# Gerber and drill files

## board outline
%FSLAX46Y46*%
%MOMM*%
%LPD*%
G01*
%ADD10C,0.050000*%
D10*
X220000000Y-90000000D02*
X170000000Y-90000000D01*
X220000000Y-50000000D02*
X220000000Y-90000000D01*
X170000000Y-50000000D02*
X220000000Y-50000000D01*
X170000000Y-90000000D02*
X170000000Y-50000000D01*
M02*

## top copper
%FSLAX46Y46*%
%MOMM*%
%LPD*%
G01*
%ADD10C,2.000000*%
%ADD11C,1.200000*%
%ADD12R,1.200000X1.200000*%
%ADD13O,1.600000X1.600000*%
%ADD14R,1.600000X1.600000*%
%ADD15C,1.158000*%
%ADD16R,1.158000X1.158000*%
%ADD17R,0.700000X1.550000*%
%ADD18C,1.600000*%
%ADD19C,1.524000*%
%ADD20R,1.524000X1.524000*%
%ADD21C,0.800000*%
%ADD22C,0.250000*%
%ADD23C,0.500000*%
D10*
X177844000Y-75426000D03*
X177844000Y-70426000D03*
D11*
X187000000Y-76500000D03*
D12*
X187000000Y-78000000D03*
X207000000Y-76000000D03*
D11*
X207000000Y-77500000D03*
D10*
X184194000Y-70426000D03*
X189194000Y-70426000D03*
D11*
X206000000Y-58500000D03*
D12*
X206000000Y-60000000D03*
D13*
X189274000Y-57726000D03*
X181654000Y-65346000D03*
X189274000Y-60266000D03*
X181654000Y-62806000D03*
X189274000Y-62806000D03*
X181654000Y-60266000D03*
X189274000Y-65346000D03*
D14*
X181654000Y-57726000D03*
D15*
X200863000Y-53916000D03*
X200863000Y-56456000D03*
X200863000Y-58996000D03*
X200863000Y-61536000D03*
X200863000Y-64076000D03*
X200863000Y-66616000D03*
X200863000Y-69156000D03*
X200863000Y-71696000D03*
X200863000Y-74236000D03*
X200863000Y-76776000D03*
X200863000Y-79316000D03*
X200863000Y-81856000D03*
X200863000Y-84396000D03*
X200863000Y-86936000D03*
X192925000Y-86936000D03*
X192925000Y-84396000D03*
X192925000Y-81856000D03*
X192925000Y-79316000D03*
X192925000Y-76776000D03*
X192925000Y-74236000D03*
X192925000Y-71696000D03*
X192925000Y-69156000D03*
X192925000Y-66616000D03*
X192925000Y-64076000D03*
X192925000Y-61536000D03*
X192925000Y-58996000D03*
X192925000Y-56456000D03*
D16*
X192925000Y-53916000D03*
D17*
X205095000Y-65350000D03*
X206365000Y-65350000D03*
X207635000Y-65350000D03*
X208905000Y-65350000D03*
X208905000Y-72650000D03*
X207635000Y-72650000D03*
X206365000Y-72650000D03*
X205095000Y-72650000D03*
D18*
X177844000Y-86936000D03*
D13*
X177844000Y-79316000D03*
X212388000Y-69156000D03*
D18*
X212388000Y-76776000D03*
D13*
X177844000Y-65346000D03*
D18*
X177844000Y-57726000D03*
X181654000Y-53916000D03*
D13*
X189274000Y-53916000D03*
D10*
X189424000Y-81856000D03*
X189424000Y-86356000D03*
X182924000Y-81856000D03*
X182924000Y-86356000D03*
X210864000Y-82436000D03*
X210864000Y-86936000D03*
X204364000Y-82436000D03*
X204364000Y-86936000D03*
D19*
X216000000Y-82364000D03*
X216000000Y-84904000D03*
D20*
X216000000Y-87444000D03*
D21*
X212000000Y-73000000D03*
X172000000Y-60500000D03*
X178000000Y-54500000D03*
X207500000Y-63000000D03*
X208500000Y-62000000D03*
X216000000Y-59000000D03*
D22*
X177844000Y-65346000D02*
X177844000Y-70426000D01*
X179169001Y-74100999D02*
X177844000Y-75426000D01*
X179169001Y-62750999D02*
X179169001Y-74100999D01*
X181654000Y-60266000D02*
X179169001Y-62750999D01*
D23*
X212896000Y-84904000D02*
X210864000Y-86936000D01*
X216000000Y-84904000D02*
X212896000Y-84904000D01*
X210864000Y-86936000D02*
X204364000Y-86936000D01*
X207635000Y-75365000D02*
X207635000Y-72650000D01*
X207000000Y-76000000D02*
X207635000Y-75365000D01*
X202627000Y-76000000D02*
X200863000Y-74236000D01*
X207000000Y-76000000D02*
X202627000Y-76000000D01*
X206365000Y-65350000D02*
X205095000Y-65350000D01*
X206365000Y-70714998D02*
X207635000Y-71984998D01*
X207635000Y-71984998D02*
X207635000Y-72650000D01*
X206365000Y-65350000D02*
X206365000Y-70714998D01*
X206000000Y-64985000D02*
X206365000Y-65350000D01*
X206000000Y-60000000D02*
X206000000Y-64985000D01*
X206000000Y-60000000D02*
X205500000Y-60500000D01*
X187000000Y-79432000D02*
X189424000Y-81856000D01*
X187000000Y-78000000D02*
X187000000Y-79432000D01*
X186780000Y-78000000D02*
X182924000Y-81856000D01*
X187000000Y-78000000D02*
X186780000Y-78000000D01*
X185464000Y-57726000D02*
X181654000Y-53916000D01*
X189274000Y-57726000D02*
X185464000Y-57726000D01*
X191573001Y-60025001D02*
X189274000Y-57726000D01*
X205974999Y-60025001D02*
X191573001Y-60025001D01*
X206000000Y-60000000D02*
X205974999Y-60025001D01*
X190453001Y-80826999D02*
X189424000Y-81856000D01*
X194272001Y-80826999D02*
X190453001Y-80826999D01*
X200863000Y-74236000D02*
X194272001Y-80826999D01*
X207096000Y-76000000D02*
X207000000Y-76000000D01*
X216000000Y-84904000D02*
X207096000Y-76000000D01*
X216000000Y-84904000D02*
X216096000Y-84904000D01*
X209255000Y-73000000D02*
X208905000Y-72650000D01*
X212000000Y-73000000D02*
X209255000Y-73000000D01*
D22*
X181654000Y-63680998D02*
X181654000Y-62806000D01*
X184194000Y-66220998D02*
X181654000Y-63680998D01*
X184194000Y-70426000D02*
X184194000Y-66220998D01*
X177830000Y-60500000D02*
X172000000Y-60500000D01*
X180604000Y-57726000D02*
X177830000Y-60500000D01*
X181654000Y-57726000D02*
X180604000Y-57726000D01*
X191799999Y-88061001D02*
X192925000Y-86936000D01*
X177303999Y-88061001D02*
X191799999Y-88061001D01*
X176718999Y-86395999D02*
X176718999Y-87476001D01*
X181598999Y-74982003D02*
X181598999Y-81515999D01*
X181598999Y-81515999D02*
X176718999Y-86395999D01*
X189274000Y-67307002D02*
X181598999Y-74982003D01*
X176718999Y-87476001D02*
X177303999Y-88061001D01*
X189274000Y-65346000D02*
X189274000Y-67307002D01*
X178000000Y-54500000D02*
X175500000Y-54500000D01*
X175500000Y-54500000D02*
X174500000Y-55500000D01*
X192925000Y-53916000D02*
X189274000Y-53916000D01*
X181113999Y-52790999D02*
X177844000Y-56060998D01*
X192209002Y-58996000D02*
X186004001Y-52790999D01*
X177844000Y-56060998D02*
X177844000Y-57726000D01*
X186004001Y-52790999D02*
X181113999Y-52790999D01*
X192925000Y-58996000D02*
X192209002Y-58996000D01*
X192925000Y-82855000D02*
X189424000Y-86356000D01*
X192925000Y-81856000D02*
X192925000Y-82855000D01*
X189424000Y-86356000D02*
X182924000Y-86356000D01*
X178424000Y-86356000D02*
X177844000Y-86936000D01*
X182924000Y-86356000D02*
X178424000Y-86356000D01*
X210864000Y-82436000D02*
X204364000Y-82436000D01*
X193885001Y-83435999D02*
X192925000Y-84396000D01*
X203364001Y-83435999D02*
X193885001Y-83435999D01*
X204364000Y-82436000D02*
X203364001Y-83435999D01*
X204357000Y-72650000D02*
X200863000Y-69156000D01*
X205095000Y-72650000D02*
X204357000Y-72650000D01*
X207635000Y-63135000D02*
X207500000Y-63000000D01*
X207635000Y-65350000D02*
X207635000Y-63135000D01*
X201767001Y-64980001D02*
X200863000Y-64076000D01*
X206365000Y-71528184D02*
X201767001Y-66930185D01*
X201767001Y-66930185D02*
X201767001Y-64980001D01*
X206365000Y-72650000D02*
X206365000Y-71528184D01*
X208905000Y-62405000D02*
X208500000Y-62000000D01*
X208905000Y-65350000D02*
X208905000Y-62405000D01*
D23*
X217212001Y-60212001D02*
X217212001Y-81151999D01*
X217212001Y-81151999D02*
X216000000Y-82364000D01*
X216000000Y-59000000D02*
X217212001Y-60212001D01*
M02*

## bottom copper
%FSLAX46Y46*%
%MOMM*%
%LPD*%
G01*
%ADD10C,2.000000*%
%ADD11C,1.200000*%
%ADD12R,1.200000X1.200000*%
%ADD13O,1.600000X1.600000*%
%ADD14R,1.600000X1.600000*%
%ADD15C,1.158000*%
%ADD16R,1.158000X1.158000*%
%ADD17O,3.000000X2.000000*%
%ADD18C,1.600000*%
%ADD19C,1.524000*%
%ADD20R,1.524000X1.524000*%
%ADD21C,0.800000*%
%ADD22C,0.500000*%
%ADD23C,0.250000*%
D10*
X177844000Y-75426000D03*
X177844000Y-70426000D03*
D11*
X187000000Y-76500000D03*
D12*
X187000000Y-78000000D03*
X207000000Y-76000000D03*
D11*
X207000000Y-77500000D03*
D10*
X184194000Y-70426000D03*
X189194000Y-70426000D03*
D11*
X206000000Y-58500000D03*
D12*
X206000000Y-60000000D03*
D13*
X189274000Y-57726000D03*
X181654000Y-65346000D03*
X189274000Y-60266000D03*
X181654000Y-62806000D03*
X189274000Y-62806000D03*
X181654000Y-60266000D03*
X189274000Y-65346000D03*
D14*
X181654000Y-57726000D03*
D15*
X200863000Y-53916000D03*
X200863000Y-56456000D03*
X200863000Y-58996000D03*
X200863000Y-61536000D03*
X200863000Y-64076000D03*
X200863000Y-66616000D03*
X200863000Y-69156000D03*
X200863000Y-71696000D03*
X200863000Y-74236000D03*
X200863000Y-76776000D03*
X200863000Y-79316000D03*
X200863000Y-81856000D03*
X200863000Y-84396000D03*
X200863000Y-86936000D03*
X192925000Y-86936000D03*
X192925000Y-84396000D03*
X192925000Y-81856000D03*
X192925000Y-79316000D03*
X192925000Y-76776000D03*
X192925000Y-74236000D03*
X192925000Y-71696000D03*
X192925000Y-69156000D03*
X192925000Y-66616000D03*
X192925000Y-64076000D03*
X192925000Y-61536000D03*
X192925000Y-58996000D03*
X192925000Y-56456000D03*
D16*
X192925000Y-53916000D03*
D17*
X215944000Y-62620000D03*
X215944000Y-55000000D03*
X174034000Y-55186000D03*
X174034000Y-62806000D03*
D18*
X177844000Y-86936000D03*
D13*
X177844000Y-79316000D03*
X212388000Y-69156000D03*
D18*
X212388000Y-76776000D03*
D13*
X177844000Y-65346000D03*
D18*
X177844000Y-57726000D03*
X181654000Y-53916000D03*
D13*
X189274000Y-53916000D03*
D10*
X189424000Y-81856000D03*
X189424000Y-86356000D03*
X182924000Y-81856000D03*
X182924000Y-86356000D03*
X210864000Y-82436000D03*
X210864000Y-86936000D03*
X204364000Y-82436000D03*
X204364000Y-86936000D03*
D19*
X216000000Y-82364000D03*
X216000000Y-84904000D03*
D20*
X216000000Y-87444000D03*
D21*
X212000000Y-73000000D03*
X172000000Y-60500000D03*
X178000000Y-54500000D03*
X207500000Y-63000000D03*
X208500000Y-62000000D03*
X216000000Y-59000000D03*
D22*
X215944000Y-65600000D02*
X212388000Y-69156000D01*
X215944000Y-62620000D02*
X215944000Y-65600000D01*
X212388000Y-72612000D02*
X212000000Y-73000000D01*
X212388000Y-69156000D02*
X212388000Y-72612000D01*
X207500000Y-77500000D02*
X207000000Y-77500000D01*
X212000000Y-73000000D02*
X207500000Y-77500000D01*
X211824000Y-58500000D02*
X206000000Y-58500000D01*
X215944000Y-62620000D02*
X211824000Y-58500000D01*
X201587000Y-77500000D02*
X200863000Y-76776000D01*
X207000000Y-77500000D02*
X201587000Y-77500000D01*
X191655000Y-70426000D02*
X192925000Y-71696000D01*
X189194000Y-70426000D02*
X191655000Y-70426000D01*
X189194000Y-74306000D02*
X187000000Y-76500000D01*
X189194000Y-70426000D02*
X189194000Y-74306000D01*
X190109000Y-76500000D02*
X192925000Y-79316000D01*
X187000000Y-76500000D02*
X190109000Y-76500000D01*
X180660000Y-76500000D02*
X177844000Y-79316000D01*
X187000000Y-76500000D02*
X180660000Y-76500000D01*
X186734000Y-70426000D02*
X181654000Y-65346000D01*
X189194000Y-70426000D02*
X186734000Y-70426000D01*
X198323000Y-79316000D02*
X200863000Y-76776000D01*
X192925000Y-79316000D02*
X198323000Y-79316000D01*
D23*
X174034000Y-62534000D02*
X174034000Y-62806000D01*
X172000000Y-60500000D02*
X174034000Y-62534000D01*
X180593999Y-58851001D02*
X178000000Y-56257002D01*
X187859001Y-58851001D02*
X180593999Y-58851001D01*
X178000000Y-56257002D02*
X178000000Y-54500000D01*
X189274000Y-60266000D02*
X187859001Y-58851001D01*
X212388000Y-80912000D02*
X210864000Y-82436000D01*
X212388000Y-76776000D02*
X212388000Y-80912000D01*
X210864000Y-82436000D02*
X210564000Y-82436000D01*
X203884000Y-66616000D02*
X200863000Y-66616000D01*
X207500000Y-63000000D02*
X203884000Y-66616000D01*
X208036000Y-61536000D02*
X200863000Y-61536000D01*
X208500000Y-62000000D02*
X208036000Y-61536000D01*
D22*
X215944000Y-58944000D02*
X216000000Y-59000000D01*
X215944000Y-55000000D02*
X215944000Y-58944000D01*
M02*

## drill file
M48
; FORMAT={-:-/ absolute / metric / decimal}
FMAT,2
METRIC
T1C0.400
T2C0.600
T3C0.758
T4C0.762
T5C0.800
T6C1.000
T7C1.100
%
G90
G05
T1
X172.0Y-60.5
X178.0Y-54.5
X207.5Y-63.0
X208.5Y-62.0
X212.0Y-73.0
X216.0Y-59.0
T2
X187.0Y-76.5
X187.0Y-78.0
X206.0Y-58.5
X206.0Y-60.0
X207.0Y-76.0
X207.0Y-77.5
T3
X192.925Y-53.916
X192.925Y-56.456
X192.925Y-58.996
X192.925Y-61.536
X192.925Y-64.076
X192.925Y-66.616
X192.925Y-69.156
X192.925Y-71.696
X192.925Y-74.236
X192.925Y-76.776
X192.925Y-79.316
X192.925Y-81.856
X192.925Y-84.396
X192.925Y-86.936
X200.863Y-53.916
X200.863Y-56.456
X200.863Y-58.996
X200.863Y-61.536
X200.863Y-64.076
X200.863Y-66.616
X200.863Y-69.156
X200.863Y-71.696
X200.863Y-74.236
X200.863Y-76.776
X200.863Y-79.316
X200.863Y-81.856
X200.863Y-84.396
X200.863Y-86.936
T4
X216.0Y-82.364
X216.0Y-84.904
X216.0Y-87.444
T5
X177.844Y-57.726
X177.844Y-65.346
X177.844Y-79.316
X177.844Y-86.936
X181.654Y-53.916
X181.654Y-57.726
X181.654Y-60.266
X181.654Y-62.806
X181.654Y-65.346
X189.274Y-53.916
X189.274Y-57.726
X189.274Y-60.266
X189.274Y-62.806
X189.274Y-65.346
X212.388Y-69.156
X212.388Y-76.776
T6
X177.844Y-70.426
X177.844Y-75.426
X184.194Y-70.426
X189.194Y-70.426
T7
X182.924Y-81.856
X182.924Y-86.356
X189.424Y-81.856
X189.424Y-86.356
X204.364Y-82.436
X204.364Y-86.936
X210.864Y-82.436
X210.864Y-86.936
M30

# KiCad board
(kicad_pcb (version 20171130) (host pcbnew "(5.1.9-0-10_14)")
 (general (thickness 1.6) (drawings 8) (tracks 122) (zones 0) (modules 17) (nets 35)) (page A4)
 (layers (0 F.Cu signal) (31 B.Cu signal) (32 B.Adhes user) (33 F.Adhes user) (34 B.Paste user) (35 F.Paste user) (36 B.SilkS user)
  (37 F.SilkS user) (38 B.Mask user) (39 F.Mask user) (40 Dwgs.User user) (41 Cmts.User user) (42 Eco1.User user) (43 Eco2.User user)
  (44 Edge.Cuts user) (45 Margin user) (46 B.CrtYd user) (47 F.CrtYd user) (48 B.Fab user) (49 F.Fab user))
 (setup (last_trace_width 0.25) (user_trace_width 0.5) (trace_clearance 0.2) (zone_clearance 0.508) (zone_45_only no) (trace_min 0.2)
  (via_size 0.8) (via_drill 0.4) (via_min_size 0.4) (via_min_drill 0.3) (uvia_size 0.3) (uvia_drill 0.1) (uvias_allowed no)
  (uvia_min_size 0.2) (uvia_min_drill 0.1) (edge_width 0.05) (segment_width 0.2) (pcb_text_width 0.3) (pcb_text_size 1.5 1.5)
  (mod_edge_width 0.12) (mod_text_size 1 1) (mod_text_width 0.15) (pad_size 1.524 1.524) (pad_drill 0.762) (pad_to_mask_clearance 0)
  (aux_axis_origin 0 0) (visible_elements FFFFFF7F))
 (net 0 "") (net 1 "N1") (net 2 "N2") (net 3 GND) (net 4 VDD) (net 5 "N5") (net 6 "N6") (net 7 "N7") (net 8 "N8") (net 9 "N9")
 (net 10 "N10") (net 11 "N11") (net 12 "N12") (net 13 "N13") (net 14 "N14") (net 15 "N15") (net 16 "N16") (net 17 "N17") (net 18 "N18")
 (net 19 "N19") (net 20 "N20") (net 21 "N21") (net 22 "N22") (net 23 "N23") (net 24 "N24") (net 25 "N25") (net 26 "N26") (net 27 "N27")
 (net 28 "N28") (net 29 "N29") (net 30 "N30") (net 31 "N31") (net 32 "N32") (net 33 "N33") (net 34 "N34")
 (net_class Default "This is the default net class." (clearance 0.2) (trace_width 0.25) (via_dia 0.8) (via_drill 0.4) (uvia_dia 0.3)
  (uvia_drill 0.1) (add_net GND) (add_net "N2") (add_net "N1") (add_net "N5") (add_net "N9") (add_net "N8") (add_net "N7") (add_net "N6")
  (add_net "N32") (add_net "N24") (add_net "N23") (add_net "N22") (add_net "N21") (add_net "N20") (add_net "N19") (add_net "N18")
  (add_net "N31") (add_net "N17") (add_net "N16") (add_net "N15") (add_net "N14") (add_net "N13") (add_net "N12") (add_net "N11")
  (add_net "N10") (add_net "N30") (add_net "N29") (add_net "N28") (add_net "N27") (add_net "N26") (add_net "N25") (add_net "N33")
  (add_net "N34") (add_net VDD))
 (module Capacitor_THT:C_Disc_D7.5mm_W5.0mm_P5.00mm (layer F.Cu) (at 177.844 70.426 270)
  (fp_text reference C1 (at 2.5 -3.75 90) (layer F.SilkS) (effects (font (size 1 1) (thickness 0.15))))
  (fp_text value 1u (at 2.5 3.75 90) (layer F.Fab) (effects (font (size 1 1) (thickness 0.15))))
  (pad 2 thru_hole circle (at 5 0 270) (size 2 2) (drill 1) (layers *.Cu *.Mask) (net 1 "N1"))
  (pad 1 thru_hole circle (at 0 0 270) (size 2 2) (drill 1) (layers *.Cu *.Mask) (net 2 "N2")))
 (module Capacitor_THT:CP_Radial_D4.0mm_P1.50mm (layer F.Cu) (at 187 78 90)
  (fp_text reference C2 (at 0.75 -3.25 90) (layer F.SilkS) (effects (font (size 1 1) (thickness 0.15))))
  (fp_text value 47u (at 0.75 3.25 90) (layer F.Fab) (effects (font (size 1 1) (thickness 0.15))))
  (pad 2 thru_hole circle (at 1.5 0 90) (size 1.2 1.2) (drill 0.6) (layers *.Cu *.Mask) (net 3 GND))
  (pad 1 thru_hole rect (at 0 0 90) (size 1.2 1.2) (drill 0.6) (layers *.Cu *.Mask) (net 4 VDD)))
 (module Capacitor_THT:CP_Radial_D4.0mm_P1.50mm (layer F.Cu) (at 207 76 270)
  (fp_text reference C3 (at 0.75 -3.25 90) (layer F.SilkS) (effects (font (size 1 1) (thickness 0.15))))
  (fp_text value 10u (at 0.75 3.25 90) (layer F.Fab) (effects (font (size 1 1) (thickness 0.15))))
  (pad 1 thru_hole rect (at 0 0 270) (size 1.2 1.2) (drill 0.6) (layers *.Cu *.Mask) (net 4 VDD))
  (pad 2 thru_hole circle (at 1.5 0 270) (size 1.2 1.2) (drill 0.6) (layers *.Cu *.Mask) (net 3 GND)))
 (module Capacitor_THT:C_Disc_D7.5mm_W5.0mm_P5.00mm (layer F.Cu) (at 184.194 70.426)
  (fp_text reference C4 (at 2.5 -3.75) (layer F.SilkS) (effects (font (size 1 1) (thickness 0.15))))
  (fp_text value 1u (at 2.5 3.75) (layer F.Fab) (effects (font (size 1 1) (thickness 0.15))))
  (pad 1 thru_hole circle (at 0 0) (size 2 2) (drill 1) (layers *.Cu *.Mask) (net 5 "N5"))
  (pad 2 thru_hole circle (at 5 0) (size 2 2) (drill 1) (layers *.Cu *.Mask) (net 3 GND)))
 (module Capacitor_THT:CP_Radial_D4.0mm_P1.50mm (layer F.Cu) (at 206 60 90)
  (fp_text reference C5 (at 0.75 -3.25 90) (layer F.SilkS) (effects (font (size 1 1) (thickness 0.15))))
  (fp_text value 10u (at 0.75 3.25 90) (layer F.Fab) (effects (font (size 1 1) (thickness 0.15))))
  (pad 2 thru_hole circle (at 1.5 0 90) (size 1.2 1.2) (drill 0.6) (layers *.Cu *.Mask) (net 3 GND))
  (pad 1 thru_hole rect (at 0 0 90) (size 1.2 1.2) (drill 0.6) (layers *.Cu *.Mask) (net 4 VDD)))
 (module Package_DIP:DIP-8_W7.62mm (layer F.Cu) (at 181.654 57.726)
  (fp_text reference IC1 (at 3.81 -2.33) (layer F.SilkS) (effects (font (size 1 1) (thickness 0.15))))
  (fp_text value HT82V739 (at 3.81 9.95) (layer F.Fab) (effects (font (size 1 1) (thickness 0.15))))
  (pad 8 thru_hole oval (at 7.62 0) (size 1.6 1.6) (drill 0.8) (layers *.Cu *.Mask) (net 4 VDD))
  (pad 4 thru_hole oval (at 0 7.62) (size 1.6 1.6) (drill 0.8) (layers *.Cu *.Mask) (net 3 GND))
  (pad 7 thru_hole oval (at 7.62 2.54) (size 1.6 1.6) (drill 0.8) (layers *.Cu *.Mask) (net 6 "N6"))
  (pad 3 thru_hole oval (at 0 5.08) (size 1.6 1.6) (drill 0.8) (layers *.Cu *.Mask) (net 5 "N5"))
  (pad 6 thru_hole oval (at 7.62 5.08) (size 1.6 1.6) (drill 0.8) (layers *.Cu *.Mask) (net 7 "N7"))
  (pad 2 thru_hole oval (at 0 2.54) (size 1.6 1.6) (drill 0.8) (layers *.Cu *.Mask) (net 1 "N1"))
  (pad 5 thru_hole oval (at 7.62 7.62) (size 1.6 1.6) (drill 0.8) (layers *.Cu *.Mask) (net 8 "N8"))
  (pad 1 thru_hole rect (at 0 0) (size 1.6 1.6) (drill 0.8) (layers *.Cu *.Mask) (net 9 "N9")))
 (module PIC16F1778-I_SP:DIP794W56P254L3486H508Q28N (layer F.Cu) (at 196.894 70.426)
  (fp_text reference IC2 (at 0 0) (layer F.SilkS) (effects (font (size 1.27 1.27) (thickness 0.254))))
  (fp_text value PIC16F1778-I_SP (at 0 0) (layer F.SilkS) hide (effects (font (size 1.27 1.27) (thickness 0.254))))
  (pad 28 thru_hole circle (at 3.969 -16.51 90) (size 1.158 1.158) (drill 0.758) (layers *.Cu *.Mask F.SilkS) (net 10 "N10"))
  (pad 27 thru_hole circle (at 3.969 -13.97 90) (size 1.158 1.158) (drill 0.758) (layers *.Cu *.Mask F.SilkS) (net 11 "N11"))
  (pad 26 thru_hole circle (at 3.969 -11.43 90) (size 1.158 1.158) (drill 0.758) (layers *.Cu *.Mask F.SilkS) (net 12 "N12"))
  (pad 25 thru_hole circle (at 3.969 -8.89 90) (size 1.158 1.158) (drill 0.758) (layers *.Cu *.Mask F.SilkS) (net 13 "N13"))
  (pad 24 thru_hole circle (at 3.969 -6.35 90) (size 1.158 1.158) (drill 0.758) (layers *.Cu *.Mask F.SilkS) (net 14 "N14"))
  (pad 23 thru_hole circle (at 3.969 -3.81 90) (size 1.158 1.158) (drill 0.758) (layers *.Cu *.Mask F.SilkS) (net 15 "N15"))
  (pad 22 thru_hole circle (at 3.969 -1.27 90) (size 1.158 1.158) (drill 0.758) (layers *.Cu *.Mask F.SilkS) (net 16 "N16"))
  (pad 21 thru_hole circle (at 3.969 1.27 90) (size 1.158 1.158) (drill 0.758) (layers *.Cu *.Mask F.SilkS) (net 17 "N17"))
  (pad 20 thru_hole circle (at 3.969 3.81 90) (size 1.158 1.158) (drill 0.758) (layers *.Cu *.Mask F.SilkS) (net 4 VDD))
  (pad 19 thru_hole circle (at 3.969 6.35 90) (size 1.158 1.158) (drill 0.758) (layers *.Cu *.Mask F.SilkS) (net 3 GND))
  (pad 18 thru_hole circle (at 3.969 8.89 90) (size 1.158 1.158) (drill 0.758) (layers *.Cu *.Mask F.SilkS) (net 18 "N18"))
  (pad 17 thru_hole circle (at 3.969 11.43 90) (size 1.158 1.158) (drill 0.758) (layers *.Cu *.Mask F.SilkS) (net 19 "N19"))
  (pad 16 thru_hole circle (at 3.969 13.97 90) (size 1.158 1.158) (drill 0.758) (layers *.Cu *.Mask F.SilkS) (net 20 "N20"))
  (pad 15 thru_hole circle (at 3.969 16.51 90) (size 1.158 1.158) (drill 0.758) (layers *.Cu *.Mask F.SilkS) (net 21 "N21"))
  (pad 14 thru_hole circle (at -3.969 16.51 90) (size 1.158 1.158) (drill 0.758) (layers *.Cu *.Mask F.SilkS) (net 8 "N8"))
  (pad 13 thru_hole circle (at -3.969 13.97 90) (size 1.158 1.158) (drill 0.758) (layers *.Cu *.Mask F.SilkS) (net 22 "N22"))
  (pad 12 thru_hole circle (at -3.969 11.43 90) (size 1.158 1.158) (drill 0.758) (layers *.Cu *.Mask F.SilkS) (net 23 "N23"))
  (pad 11 thru_hole circle (at -3.969 8.89 90) (size 1.158 1.158) (drill 0.758) (layers *.Cu *.Mask F.SilkS) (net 3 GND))
  (pad 10 thru_hole circle (at -3.969 6.35 90) (size 1.158 1.158) (drill 0.758) (layers *.Cu *.Mask F.SilkS) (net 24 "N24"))
  (pad 9 thru_hole circle (at -3.969 3.81 90) (size 1.158 1.158) (drill 0.758) (layers *.Cu *.Mask F.SilkS) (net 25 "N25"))
  (pad 8 thru_hole circle (at -3.969 1.27 90) (size 1.158 1.158) (drill 0.758) (layers *.Cu *.Mask F.SilkS) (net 3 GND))
  (pad 7 thru_hole circle (at -3.969 -1.27 90) (size 1.158 1.158) (drill 0.758) (layers *.Cu *.Mask F.SilkS) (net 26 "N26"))
  (pad 6 thru_hole circle (at -3.969 -3.81 90) (size 1.158 1.158) (drill 0.758) (layers *.Cu *.Mask F.SilkS) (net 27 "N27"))
  (pad 5 thru_hole circle (at -3.969 -6.35 90) (size 1.158 1.158) (drill 0.758) (layers *.Cu *.Mask F.SilkS) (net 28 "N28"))
  (pad 4 thru_hole circle (at -3.969 -8.89 90) (size 1.158 1.158) (drill 0.758) (layers *.Cu *.Mask F.SilkS) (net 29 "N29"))
  (pad 3 thru_hole circle (at -3.969 -11.43 90) (size 1.158 1.158) (drill 0.758) (layers *.Cu *.Mask F.SilkS) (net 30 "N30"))
  (pad 2 thru_hole circle (at -3.969 -13.97 90) (size 1.158 1.158) (drill 0.758) (layers *.Cu *.Mask F.SilkS) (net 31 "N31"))
  (pad 1 thru_hole rect (at -3.969 -16.51 90) (size 1.158 1.158) (drill 0.758) (layers *.Cu *.Mask F.SilkS) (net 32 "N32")))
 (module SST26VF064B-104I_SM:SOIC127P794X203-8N (layer F.Cu) (at 207 69 90)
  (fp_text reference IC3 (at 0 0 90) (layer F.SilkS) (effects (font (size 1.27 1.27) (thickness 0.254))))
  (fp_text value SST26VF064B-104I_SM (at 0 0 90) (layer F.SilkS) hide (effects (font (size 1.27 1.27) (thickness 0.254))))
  (pad 8 smd rect (at 3.65 -1.905 180) (size 0.7 1.55) (layers F.Cu F.Paste F.Mask) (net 4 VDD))
  (pad 7 smd rect (at 3.65 -0.635 180) (size 0.7 1.55) (layers F.Cu F.Paste F.Mask) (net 4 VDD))
  (pad 6 smd rect (at 3.65 0.635 180) (size 0.7 1.55) (layers F.Cu F.Paste F.Mask) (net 15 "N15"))
  (pad 5 smd rect (at 3.65 1.905 180) (size 0.7 1.55) (layers F.Cu F.Paste F.Mask) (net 13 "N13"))
  (pad 4 smd rect (at -3.65 1.905 180) (size 0.7 1.55) (layers F.Cu F.Paste F.Mask) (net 3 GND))
  (pad 3 smd rect (at -3.65 0.635 180) (size 0.7 1.55) (layers F.Cu F.Paste F.Mask) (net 4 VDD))
  (pad 2 smd rect (at -3.65 -0.635 180) (size 0.7 1.55) (layers F.Cu F.Paste F.Mask) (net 14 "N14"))
  (pad 1 smd rect (at -3.65 -1.905 180) (size 0.7 1.55) (layers F.Cu F.Paste F.Mask) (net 16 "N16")))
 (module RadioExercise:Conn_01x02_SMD (layer B.Cu) (at 215.944 58.81 90)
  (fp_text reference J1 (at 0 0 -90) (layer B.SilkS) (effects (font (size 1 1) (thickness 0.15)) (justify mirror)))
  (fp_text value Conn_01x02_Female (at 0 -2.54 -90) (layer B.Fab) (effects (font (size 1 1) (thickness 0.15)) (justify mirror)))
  (pad 1 smd oval (at -3.81 0 90) (size 2 3) (layers B.Cu B.Paste B.Mask) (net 3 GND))
  (pad 2 smd oval (at 3.81 0 90) (size 2 3) (layers B.Cu B.Paste B.Mask) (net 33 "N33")))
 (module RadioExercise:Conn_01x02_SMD (layer B.Cu) (at 174.034 58.996 90)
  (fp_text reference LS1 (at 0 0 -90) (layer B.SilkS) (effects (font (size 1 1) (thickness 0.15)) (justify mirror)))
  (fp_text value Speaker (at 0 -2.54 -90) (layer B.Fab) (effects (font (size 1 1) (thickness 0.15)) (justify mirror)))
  (pad 2 smd oval (at 3.81 0 90) (size 2 3) (layers B.Cu B.Paste B.Mask) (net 6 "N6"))
  (pad 1 smd oval (at -3.81 0 90) (size 2 3) (layers B.Cu B.Paste B.Mask) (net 9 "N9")))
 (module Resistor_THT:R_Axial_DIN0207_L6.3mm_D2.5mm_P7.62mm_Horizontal (layer F.Cu) (at 177.844 86.936 90)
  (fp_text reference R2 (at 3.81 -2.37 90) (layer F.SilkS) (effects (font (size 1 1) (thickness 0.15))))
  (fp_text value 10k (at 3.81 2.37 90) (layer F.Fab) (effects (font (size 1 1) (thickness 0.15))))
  (pad 1 thru_hole circle (at 0 0 90) (size 1.6 1.6) (drill 0.8) (layers *.Cu *.Mask) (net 23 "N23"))
  (pad 2 thru_hole oval (at 7.62 0 90) (size 1.6 1.6) (drill 0.8) (layers *.Cu *.Mask) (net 3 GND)))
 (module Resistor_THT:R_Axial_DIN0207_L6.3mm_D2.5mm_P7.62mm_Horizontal (layer F.Cu) (at 212.388 76.776 90)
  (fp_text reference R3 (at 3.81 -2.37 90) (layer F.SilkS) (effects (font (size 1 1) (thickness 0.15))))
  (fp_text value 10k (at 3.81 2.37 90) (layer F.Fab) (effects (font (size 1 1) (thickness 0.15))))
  (pad 2 thru_hole oval (at 7.62 0 90) (size 1.6 1.6) (drill 0.8) (layers *.Cu *.Mask) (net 3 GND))
  (pad 1 thru_hole circle (at 0 0 90) (size 1.6 1.6) (drill 0.8) (layers *.Cu *.Mask) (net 22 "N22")))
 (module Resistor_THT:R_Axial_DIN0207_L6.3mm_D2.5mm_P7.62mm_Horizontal (layer F.Cu) (at 177.844 57.726 270)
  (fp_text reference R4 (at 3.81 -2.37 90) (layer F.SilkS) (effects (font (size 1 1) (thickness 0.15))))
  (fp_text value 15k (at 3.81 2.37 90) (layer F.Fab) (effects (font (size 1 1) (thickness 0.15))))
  (pad 2 thru_hole oval (at 7.62 0 270) (size 1.6 1.6) (drill 0.8) (layers *.Cu *.Mask) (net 2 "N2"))
  (pad 1 thru_hole circle (at 0 0 270) (size 1.6 1.6) (drill 0.8) (layers *.Cu *.Mask) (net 30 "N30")))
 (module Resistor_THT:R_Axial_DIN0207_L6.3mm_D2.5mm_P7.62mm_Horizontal (layer F.Cu) (at 181.654 53.916)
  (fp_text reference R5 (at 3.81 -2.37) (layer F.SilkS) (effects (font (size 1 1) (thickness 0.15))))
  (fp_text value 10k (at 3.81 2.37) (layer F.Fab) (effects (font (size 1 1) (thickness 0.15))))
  (pad 1 thru_hole circle (at 0 0) (size 1.6 1.6) (drill 0.8) (layers *.Cu *.Mask) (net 4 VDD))
  (pad 2 thru_hole oval (at 7.62 0) (size 1.6 1.6) (drill 0.8) (layers *.Cu *.Mask) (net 32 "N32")))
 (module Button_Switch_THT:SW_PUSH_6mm (layer F.Cu) (at 182.924 81.856)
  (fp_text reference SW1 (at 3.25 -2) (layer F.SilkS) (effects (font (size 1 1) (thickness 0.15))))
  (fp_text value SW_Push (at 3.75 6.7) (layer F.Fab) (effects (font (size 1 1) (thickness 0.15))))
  (pad 1 thru_hole circle (at 6.5 0 90) (size 2 2) (drill 1.1) (layers *.Cu *.Mask) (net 4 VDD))
  (pad 2 thru_hole circle (at 6.5 4.5 90) (size 2 2) (drill 1.1) (layers *.Cu *.Mask) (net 23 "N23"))
  (pad 1 thru_hole circle (at 0 0 90) (size 2 2) (drill 1.1) (layers *.Cu *.Mask) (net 4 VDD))
  (pad 2 thru_hole circle (at 0 4.5 90) (size 2 2) (drill 1.1) (layers *.Cu *.Mask) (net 23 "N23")))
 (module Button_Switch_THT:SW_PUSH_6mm (layer F.Cu) (at 210.864 86.936 180)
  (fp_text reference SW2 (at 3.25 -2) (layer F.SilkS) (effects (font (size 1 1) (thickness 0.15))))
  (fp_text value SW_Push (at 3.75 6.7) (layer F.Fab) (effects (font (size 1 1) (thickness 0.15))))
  (pad 2 thru_hole circle (at 0 4.5 270) (size 2 2) (drill 1.1) (layers *.Cu *.Mask) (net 22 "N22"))
  (pad 1 thru_hole circle (at 0 0 270) (size 2 2) (drill 1.1) (layers *.Cu *.Mask) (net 4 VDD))
  (pad 2 thru_hole circle (at 6.5 4.5 270) (size 2 2) (drill 1.1) (layers *.Cu *.Mask) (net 22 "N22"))
  (pad 1 thru_hole circle (at 6.5 0 270) (size 2 2) (drill 1.1) (layers *.Cu *.Mask) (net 4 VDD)))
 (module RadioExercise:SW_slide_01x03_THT (layer F.Cu) (at 216 84.904 90)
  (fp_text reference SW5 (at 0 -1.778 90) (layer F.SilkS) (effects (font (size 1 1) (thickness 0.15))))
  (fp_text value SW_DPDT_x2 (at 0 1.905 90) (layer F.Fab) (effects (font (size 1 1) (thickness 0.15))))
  (pad 3 thru_hole circle (at 2.54 0 90) (size 1.524 1.524) (drill 0.762) (layers *.Cu *.Mask) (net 33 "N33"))
  (pad 2 thru_hole circle (at 0 0 90) (size 1.524 1.524) (drill 0.762) (layers *.Cu *.Mask) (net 4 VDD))
  (pad 1 thru_hole rect (at -2.54 0 90) (size 1.524 1.524) (drill 0.762) (layers *.Cu *.Mask) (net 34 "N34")))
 (gr_line (start 220 90) (end 170 90) (layer Edge.Cuts) (width 0.05))
 (gr_line (start 220 50) (end 220 90) (layer Edge.Cuts) (width 0.05))
 (gr_line (start 170 50) (end 220 50) (layer Edge.Cuts) (width 0.05))
 (gr_line (start 170 90) (end 170 50) (layer Edge.Cuts) (width 0.05))
 (segment (start 177.844 65.346) (end 177.844 70.426) (width 0.25) (layer F.Cu) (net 2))
 (segment (start 179.169001 74.100999) (end 177.844 75.426) (width 0.25) (layer F.Cu) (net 1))
 (segment (start 179.169001 62.750999) (end 179.169001 74.100999) (width 0.25) (layer F.Cu) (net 1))
 (segment (start 181.654 60.266) (end 179.169001 62.750999) (width 0.25) (layer F.Cu) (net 1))
 (segment (start 212.896 84.904) (end 210.864 86.936) (width 0.5) (layer F.Cu) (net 4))
 (segment (start 216 84.904) (end 212.896 84.904) (width 0.5) (layer F.Cu) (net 4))
 (segment (start 210.864 86.936) (end 204.364 86.936) (width 0.5) (layer F.Cu) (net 4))
 (segment (start 207.635 75.365) (end 207.635 72.65) (width 0.5) (layer F.Cu) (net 4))
 (segment (start 207 76) (end 207.635 75.365) (width 0.5) (layer F.Cu) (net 4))
 (segment (start 202.627 76) (end 200.863 74.236) (width 0.5) (layer F.Cu) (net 4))
 (segment (start 207 76) (end 202.627 76) (width 0.5) (layer F.Cu) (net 4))
 (segment (start 206.365 65.35) (end 205.095 65.35) (width 0.5) (layer F.Cu) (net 4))
 (segment (start 206.365 70.714998) (end 207.635 71.984998) (width 0.5) (layer F.Cu) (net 4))
 (segment (start 207.635 71.984998) (end 207.635 72.65) (width 0.5) (layer F.Cu) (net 4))
 (segment (start 206.365 65.35) (end 206.365 70.714998) (width 0.5) (layer F.Cu) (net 4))
 (segment (start 206 64.985) (end 206.365 65.35) (width 0.5) (layer F.Cu) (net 4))
 (segment (start 206 60) (end 206 64.985) (width 0.5) (layer F.Cu) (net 4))
 (segment (start 206 60) (end 205.5 60.5) (width 0.5) (layer F.Cu) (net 4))
 (segment (start 187 79.432) (end 189.424 81.856) (width 0.5) (layer F.Cu) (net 4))
 (segment (start 187 78) (end 187 79.432) (width 0.5) (layer F.Cu) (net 4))
 (segment (start 186.78 78) (end 182.924 81.856) (width 0.5) (layer F.Cu) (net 4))
 (segment (start 187 78) (end 186.78 78) (width 0.5) (layer F.Cu) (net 4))
 (segment (start 185.464 57.726) (end 181.654 53.916) (width 0.5) (layer F.Cu) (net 4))
 (segment (start 189.274 57.726) (end 185.464 57.726) (width 0.5) (layer F.Cu) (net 4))
 (segment (start 191.573001 60.025001) (end 189.274 57.726) (width 0.5) (layer F.Cu) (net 4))
 (segment (start 205.974999 60.025001) (end 191.573001 60.025001) (width 0.5) (layer F.Cu) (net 4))
 (segment (start 206 60) (end 205.974999 60.025001) (width 0.5) (layer F.Cu) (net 4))
 (segment (start 190.453001 80.826999) (end 189.424 81.856) (width 0.5) (layer F.Cu) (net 4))
 (segment (start 194.272001 80.826999) (end 190.453001 80.826999) (width 0.5) (layer F.Cu) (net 4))
 (segment (start 200.863 74.236) (end 194.272001 80.826999) (width 0.5) (layer F.Cu) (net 4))
 (segment (start 207.096 76) (end 207 76) (width 0.5) (layer F.Cu) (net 4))
 (segment (start 216 84.904) (end 207.096 76) (width 0.5) (layer F.Cu) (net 4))
 (segment (start 216 84.904) (end 216.096 84.904) (width 0.5) (layer F.Cu) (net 4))
 (segment (start 215.944 65.6) (end 212.388 69.156) (width 0.5) (layer B.Cu) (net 3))
 (segment (start 215.944 62.62) (end 215.944 65.6) (width 0.5) (layer B.Cu) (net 3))
 (via (at 212 73) (size 0.8) (drill 0.4) (layers F.Cu B.Cu) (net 3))
 (segment (start 212.388 72.612) (end 212 73) (width 0.5) (layer B.Cu) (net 3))
 (segment (start 212.388 69.156) (end 212.388 72.612) (width 0.5) (layer B.Cu) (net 3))
 (segment (start 209.255 73) (end 208.905 72.65) (width 0.5) (layer F.Cu) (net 3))
 (segment (start 212 73) (end 209.255 73) (width 0.5) (layer F.Cu) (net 3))
 (segment (start 207.5 77.5) (end 207 77.5) (width 0.5) (layer B.Cu) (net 3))
 (segment (start 212 73) (end 207.5 77.5) (width 0.5) (layer B.Cu) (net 3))
 (segment (start 211.824 58.5) (end 206 58.5) (width 0.5) (layer B.Cu) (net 3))
 (segment (start 215.944 62.62) (end 211.824 58.5) (width 0.5) (layer B.Cu) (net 3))
 (segment (start 201.587 77.5) (end 200.863 76.776) (width 0.5) (layer B.Cu) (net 3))
 (segment (start 207 77.5) (end 201.587 77.5) (width 0.5) (layer B.Cu) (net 3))
 (segment (start 191.655 70.426) (end 192.925 71.696) (width 0.5) (layer B.Cu) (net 3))
 (segment (start 189.194 70.426) (end 191.655 70.426) (width 0.5) (layer B.Cu) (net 3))
 (segment (start 189.194 74.306) (end 187 76.5) (width 0.5) (layer B.Cu) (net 3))
 (segment (start 189.194 70.426) (end 189.194 74.306) (width 0.5) (layer B.Cu) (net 3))
 (segment (start 190.109 76.5) (end 192.925 79.316) (width 0.5) (layer B.Cu) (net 3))
 (segment (start 187 76.5) (end 190.109 76.5) (width 0.5) (layer B.Cu) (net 3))
 (segment (start 180.66 76.5) (end 177.844 79.316) (width 0.5) (layer B.Cu) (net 3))
 (segment (start 187 76.5) (end 180.66 76.5) (width 0.5) (layer B.Cu) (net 3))
 (segment (start 186.734 70.426) (end 181.654 65.346) (width 0.5) (layer B.Cu) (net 3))
 (segment (start 189.194 70.426) (end 186.734 70.426) (width 0.5) (layer B.Cu) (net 3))
 (segment (start 198.323 79.316) (end 200.863 76.776) (width 0.5) (layer B.Cu) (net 3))
 (segment (start 192.925 79.316) (end 198.323 79.316) (width 0.5) (layer B.Cu) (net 3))
 (segment (start 181.654 63.680998) (end 181.654 62.806) (width 0.25) (layer F.Cu) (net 5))
 (segment (start 184.194 66.220998) (end 181.654 63.680998) (width 0.25) (layer F.Cu) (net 5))
 (segment (start 184.194 70.426) (end 184.194 66.220998) (width 0.25) (layer F.Cu) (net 5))
 (via (at 172 60.5) (size 0.8) (drill 0.4) (layers F.Cu B.Cu) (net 9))
 (segment (start 177.83 60.5) (end 172 60.5) (width 0.25) (layer F.Cu) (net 9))
 (segment (start 180.604 57.726) (end 177.83 60.5) (width 0.25) (layer F.Cu) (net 9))
 (segment (start 181.654 57.726) (end 180.604 57.726) (width 0.25) (layer F.Cu) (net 9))
 (segment (start 174.034 62.534) (end 174.034 62.806) (width 0.25) (layer B.Cu) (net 9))
 (segment (start 172 60.5) (end 174.034 62.534) (width 0.25) (layer B.Cu) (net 9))
 (segment (start 191.799999 88.061001) (end 192.925 86.936) (width 0.25) (layer F.Cu) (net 8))
 (segment (start 177.303999 88.061001) (end 191.799999 88.061001) (width 0.25) (layer F.Cu) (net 8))
 (segment (start 176.718999 86.395999) (end 176.718999 87.476001) (width 0.25) (layer F.Cu) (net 8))
 (segment (start 181.598999 74.982003) (end 181.598999 81.515999) (width 0.25) (layer F.Cu) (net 8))
 (segment (start 181.598999 81.515999) (end 176.718999 86.395999) (width 0.25) (layer F.Cu) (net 8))
 (segment (start 189.274 67.307002) (end 181.598999 74.982003) (width 0.25) (layer F.Cu) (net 8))
 (segment (start 176.718999 87.476001) (end 177.303999 88.061001) (width 0.25) (layer F.Cu) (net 8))
 (segment (start 189.274 65.346) (end 189.274 67.307002) (width 0.25) (layer F.Cu) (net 8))
 (segment (start 180.593999 58.851001) (end 178 56.257002) (width 0.25) (layer B.Cu) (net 6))
 (via (at 178 54.5) (size 0.8) (drill 0.4) (layers F.Cu B.Cu) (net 6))
 (segment (start 187.859001 58.851001) (end 180.593999 58.851001) (width 0.25) (layer B.Cu) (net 6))
 (segment (start 178 56.257002) (end 178 54.5) (width 0.25) (layer B.Cu) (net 6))
 (segment (start 189.274 60.266) (end 187.859001 58.851001) (width 0.25) (layer B.Cu) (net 6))
 (segment (start 178 54.5) (end 175.5 54.5) (width 0.25) (layer F.Cu) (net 6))
 (segment (start 175.5 54.5) (end 174.5 55.5) (width 0.25) (layer F.Cu) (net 6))
 (segment (start 192.925 53.916) (end 189.274 53.916) (width 0.25) (layer F.Cu) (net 32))
 (segment (start 181.113999 52.790999) (end 177.844 56.060998) (width 0.25) (layer F.Cu) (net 30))
 (segment (start 192.209002 58.996) (end 186.004001 52.790999) (width 0.25) (layer F.Cu) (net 30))
 (segment (start 177.844 56.060998) (end 177.844 57.726) (width 0.25) (layer F.Cu) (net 30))
 (segment (start 186.004001 52.790999) (end 181.113999 52.790999) (width 0.25) (layer F.Cu) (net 30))
 (segment (start 192.925 58.996) (end 192.209002 58.996) (width 0.25) (layer F.Cu) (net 30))
 (segment (start 192.925 82.855) (end 189.424 86.356) (width 0.25) (layer F.Cu) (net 23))
 (segment (start 192.925 81.856) (end 192.925 82.855) (width 0.25) (layer F.Cu) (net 23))
 (segment (start 189.424 86.356) (end 182.924 86.356) (width 0.25) (layer F.Cu) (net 23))
 (segment (start 178.424 86.356) (end 177.844 86.936) (width 0.25) (layer F.Cu) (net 23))
 (segment (start 182.924 86.356) (end 178.424 86.356) (width 0.25) (layer F.Cu) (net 23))
 (segment (start 212.388 80.912) (end 210.864 82.436) (width 0.25) (layer B.Cu) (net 22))
 (segment (start 212.388 76.776) (end 212.388 80.912) (width 0.25) (layer B.Cu) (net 22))
 (segment (start 210.864 82.436) (end 210.564 82.436) (width 0.25) (layer B.Cu) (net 22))
 (segment (start 210.864 82.436) (end 204.364 82.436) (width 0.25) (layer F.Cu) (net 22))
 (segment (start 193.885001 83.435999) (end 192.925 84.396) (width 0.25) (layer F.Cu) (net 22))
 (segment (start 203.364001 83.435999) (end 193.885001 83.435999) (width 0.25) (layer F.Cu) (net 22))
 (segment (start 204.364 82.436) (end 203.364001 83.435999) (width 0.25) (layer F.Cu) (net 22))
 (segment (start 204.357 72.65) (end 200.863 69.156) (width 0.25) (layer F.Cu) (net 16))
 (segment (start 205.095 72.65) (end 204.357 72.65) (width 0.25) (layer F.Cu) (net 16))
 (via (at 207.5 63) (size 0.8) (drill 0.4) (layers F.Cu B.Cu) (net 15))
 (segment (start 207.635 63.135) (end 207.5 63) (width 0.25) (layer F.Cu) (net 15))
 (segment (start 207.635 65.35) (end 207.635 63.135) (width 0.25) (layer F.Cu) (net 15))
 (segment (start 203.884 66.616) (end 200.863 66.616) (width 0.25) (layer B.Cu) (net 15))
 (segment (start 207.5 63) (end 203.884 66.616) (width 0.25) (layer B.Cu) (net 15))
 (segment (start 201.767001 64.980001) (end 200.863 64.076) (width 0.25) (layer F.Cu) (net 14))
 (segment (start 206.365 71.528184) (end 201.767001 66.930185) (width 0.25) (layer F.Cu) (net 14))
 (segment (start 201.767001 66.930185) (end 201.767001 64.980001) (width 0.25) (layer F.Cu) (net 14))
 (segment (start 206.365 72.65) (end 206.365 71.528184) (width 0.25) (layer F.Cu) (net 14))
 (via (at 208.5 62) (size 0.8) (drill 0.4) (layers F.Cu B.Cu) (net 13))
 (segment (start 208.905 62.405) (end 208.5 62) (width 0.25) (layer F.Cu) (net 13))
 (segment (start 208.905 65.35) (end 208.905 62.405) (width 0.25) (layer F.Cu) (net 13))
 (segment (start 208.036 61.536) (end 200.863 61.536) (width 0.25) (layer B.Cu) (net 13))
 (segment (start 208.5 62) (end 208.036 61.536) (width 0.25) (layer B.Cu) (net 13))
 (via (at 216 59) (size 0.8) (drill 0.4) (layers F.Cu B.Cu) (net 33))
 (segment (start 215.944 58.944) (end 216 59) (width 0.5) (layer B.Cu) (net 33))
 (segment (start 215.944 55) (end 215.944 58.944) (width 0.5) (layer B.Cu) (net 33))
 (segment (start 217.212001 60.212001) (end 217.212001 81.151999) (width 0.5) (layer F.Cu) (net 33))
 (segment (start 217.212001 81.151999) (end 216 82.364) (width 0.5) (layer F.Cu) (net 33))
 (segment (start 216 59) (end 217.212001 60.212001) (width 0.5) (layer F.Cu) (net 33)))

